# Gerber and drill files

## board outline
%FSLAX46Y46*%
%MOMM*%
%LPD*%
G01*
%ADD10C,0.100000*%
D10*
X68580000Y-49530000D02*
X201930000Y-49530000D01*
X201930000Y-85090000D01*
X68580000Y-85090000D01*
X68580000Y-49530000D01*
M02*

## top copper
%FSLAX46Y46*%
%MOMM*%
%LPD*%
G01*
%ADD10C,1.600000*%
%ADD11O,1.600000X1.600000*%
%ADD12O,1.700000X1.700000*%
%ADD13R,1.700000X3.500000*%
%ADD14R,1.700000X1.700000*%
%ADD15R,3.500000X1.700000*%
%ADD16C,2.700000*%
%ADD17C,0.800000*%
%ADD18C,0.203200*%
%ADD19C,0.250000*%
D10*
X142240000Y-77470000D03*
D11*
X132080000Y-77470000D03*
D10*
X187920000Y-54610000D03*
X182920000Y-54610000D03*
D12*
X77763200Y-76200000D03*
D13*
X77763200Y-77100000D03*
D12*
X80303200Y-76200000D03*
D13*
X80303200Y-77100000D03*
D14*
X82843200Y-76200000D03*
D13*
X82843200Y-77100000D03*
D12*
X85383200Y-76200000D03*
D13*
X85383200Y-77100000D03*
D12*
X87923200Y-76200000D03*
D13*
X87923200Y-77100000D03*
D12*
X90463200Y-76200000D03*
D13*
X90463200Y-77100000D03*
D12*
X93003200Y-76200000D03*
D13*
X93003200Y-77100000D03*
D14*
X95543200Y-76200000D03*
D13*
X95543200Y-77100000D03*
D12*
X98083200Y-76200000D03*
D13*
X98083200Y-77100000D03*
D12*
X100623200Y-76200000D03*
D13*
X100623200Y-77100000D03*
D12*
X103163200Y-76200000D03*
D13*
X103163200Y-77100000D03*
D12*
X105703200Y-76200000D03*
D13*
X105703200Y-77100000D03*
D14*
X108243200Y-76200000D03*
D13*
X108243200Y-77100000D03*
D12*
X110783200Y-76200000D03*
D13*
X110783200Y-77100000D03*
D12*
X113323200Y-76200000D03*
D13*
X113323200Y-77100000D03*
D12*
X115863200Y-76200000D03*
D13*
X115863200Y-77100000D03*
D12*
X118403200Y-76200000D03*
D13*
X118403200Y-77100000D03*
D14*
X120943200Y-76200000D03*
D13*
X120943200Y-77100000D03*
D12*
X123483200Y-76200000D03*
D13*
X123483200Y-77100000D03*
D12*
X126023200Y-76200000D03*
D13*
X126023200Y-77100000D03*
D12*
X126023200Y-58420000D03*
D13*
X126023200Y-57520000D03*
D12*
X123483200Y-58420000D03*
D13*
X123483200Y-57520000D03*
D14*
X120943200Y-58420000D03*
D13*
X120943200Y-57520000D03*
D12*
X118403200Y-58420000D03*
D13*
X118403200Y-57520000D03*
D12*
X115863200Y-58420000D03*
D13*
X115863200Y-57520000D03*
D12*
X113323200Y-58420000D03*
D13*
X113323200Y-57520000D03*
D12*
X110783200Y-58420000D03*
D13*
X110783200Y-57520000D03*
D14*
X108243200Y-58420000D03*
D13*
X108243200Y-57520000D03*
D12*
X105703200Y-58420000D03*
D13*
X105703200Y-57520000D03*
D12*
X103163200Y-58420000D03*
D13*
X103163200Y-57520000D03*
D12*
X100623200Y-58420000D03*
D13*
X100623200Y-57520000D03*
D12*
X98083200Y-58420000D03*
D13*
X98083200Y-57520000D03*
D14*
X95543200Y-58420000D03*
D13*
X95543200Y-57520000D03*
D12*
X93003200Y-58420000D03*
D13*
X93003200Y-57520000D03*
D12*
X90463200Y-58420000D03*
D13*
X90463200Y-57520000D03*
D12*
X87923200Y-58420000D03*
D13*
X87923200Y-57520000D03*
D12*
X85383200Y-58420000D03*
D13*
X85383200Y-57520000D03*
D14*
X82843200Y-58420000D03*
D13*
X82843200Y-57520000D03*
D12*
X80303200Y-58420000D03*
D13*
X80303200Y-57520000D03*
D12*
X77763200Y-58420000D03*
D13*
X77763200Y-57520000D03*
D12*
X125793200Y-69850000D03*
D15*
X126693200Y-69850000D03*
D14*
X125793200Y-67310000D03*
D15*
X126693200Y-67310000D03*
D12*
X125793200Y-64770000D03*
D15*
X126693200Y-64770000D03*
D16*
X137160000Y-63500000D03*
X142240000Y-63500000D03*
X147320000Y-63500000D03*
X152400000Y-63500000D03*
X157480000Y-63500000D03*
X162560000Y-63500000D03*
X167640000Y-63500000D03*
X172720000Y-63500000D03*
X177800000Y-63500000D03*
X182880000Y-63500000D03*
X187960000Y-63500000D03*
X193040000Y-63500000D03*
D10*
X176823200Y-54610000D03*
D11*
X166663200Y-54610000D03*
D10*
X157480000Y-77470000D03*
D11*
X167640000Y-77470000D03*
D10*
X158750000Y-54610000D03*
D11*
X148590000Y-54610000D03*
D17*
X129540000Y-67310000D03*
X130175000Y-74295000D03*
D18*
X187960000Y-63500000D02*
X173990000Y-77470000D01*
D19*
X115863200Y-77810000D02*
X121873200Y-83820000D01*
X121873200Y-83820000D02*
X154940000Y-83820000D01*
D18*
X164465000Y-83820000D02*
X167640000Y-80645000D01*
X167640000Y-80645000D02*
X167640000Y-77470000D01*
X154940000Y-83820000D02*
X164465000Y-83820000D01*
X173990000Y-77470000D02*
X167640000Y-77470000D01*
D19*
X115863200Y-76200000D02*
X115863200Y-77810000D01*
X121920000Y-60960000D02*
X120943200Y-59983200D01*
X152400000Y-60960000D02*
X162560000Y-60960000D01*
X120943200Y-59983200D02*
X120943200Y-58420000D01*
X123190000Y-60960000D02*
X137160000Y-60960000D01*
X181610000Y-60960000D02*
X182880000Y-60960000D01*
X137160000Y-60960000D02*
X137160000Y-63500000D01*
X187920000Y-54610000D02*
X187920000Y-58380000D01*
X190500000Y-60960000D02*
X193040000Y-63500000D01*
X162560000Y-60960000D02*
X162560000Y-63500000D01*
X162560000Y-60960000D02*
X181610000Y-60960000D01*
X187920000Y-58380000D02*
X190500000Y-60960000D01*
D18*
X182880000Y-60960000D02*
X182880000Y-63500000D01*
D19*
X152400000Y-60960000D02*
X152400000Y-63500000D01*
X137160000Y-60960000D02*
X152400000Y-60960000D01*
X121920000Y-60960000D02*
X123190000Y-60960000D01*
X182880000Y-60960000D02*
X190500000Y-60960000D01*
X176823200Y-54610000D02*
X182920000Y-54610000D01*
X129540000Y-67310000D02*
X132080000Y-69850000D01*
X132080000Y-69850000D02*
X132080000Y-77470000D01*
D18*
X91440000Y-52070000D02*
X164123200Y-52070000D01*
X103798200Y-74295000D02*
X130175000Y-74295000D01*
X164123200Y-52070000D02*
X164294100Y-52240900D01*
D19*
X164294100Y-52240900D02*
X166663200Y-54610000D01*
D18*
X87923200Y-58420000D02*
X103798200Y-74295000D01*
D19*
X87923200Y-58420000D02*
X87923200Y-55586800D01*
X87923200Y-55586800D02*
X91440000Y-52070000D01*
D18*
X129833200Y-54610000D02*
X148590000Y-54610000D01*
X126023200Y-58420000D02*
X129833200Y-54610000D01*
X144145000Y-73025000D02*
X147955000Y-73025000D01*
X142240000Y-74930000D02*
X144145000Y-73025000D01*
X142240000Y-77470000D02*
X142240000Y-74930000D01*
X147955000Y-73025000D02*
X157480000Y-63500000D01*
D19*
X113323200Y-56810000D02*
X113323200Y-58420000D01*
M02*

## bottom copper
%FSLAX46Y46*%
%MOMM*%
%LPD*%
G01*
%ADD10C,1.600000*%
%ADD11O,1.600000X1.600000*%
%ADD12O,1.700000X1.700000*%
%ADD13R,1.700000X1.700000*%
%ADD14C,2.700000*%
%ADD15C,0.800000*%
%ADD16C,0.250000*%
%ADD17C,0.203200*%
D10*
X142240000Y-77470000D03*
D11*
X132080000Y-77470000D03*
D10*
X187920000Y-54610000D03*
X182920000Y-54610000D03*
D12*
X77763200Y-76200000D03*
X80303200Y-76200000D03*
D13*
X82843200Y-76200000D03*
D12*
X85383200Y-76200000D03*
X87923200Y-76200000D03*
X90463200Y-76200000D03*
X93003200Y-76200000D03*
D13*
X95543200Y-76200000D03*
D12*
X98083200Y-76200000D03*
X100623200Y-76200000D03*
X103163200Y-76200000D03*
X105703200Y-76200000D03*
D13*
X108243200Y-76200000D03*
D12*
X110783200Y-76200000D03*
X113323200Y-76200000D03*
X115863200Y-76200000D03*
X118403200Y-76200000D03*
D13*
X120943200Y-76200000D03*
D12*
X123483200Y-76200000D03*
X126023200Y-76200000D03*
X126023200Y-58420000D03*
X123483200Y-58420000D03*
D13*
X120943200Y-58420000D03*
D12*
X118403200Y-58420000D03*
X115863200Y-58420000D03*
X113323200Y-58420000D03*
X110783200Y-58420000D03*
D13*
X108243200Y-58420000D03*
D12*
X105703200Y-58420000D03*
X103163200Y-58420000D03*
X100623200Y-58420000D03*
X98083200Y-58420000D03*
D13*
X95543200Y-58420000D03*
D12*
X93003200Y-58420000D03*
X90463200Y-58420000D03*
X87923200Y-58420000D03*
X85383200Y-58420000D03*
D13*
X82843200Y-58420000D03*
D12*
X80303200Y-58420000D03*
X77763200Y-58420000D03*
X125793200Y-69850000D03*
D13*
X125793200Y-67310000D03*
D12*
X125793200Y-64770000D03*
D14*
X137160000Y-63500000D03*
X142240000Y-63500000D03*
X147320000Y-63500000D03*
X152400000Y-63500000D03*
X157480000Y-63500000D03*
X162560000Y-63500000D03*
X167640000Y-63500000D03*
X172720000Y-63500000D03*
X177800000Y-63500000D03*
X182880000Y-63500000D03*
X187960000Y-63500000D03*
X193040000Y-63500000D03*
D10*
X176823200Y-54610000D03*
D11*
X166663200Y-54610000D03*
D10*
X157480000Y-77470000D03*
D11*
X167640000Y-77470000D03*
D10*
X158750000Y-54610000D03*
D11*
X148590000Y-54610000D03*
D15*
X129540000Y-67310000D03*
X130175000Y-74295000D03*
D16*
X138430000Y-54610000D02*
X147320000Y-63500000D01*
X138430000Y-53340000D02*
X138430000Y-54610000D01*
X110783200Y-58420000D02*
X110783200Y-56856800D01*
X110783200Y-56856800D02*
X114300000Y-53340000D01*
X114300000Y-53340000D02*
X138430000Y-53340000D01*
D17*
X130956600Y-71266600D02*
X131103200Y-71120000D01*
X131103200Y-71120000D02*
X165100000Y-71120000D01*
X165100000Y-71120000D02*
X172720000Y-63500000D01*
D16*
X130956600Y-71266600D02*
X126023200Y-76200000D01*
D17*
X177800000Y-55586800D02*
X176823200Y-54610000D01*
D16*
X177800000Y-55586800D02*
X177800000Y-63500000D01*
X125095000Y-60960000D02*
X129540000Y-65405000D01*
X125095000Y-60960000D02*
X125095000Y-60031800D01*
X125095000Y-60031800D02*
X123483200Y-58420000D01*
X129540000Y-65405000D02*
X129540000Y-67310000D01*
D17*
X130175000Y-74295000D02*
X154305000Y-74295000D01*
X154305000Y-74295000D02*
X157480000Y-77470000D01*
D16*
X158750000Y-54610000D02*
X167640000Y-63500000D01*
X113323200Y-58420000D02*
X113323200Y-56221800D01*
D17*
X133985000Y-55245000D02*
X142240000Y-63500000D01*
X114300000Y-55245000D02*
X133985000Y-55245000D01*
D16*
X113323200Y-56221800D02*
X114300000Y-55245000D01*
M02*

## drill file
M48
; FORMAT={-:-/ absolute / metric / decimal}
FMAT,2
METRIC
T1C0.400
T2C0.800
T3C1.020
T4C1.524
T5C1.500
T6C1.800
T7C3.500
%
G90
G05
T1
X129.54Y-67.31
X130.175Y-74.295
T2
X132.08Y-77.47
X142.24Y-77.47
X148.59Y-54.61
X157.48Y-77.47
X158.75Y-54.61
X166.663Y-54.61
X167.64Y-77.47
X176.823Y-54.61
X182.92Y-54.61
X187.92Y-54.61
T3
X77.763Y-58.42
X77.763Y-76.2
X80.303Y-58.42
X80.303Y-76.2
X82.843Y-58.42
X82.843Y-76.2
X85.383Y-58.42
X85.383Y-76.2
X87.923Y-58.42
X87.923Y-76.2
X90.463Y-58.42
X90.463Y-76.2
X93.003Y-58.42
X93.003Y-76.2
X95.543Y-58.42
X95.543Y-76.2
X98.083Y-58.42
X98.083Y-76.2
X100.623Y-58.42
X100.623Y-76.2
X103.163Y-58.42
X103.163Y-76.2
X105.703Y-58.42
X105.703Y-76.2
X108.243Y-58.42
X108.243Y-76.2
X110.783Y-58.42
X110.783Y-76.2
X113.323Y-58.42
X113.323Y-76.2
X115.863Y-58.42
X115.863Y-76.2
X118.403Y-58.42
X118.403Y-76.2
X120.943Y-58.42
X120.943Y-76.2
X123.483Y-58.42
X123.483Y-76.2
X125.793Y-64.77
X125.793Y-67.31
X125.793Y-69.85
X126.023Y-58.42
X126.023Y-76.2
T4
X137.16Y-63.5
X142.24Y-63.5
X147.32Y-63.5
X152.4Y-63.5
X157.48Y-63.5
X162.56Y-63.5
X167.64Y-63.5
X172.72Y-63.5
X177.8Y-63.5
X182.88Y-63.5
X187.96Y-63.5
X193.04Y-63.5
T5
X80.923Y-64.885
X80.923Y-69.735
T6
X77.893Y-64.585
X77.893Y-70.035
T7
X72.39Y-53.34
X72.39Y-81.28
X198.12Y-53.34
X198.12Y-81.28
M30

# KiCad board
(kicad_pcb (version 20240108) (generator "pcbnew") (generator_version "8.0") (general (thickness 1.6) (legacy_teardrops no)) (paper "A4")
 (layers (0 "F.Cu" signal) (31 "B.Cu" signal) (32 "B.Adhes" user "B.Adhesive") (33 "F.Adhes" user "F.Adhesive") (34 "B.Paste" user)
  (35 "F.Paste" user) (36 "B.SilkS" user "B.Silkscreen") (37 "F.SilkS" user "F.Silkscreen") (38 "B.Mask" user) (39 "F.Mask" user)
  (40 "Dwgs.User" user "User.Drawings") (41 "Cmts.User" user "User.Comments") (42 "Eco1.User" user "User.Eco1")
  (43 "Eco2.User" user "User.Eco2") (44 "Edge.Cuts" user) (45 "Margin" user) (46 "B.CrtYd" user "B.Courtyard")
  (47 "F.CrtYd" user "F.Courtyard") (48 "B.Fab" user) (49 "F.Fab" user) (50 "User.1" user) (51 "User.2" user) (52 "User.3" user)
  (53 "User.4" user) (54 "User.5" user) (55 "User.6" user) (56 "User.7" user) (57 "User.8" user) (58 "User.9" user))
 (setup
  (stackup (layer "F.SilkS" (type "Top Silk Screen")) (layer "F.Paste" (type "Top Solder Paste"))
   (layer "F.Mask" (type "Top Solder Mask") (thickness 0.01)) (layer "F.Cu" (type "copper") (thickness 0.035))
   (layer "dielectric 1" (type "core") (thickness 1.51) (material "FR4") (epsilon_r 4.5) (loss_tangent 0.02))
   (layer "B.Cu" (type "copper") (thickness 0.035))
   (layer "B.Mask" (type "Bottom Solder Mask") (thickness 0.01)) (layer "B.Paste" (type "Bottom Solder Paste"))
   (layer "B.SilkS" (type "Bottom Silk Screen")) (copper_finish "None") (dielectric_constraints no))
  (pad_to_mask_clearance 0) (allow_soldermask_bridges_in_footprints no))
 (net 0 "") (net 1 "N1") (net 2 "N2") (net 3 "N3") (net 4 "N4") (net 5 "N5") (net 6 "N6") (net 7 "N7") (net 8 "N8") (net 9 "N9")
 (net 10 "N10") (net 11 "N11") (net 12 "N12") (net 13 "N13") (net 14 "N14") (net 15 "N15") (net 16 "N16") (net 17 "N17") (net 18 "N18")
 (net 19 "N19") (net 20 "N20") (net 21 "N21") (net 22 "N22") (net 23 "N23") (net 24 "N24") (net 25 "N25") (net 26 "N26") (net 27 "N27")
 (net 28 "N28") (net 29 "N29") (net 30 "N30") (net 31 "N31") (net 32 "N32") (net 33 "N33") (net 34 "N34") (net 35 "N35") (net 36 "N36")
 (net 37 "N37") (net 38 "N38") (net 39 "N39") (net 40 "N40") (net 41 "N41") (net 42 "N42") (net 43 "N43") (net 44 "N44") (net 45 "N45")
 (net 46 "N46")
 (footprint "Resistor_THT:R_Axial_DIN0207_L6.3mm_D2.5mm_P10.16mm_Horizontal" (layer "F.Cu") (at 142.24 77.47 180)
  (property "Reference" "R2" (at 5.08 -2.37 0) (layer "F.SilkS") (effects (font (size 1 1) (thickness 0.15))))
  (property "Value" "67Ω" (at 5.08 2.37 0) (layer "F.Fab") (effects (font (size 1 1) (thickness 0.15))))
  (pad "1" thru_hole circle (at 0 0 180) (size 1.6 1.6) (drill 0.8) (layers "*.Cu" "*.Mask") (remove_unused_layers no) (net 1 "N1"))
  (pad "2" thru_hole oval (at 10.16 0 180) (size 1.6 1.6) (drill 0.8) (layers "*.Cu" "*.Mask") (remove_unused_layers no) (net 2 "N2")))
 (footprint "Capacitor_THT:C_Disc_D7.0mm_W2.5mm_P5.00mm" (layer "F.Cu") (at 187.92 54.61 180)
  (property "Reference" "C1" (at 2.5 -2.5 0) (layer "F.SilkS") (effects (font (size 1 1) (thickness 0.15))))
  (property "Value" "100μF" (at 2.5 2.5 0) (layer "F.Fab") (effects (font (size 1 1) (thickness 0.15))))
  (pad "1" thru_hole circle (at 0 0 180) (size 1.6 1.6) (drill 0.8) (layers "*.Cu" "*.Mask") (remove_unused_layers no) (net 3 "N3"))
  (pad "2" thru_hole circle (at 5 0 180) (size 1.6 1.6) (drill 0.8) (layers "*.Cu" "*.Mask") (remove_unused_layers no) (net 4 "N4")))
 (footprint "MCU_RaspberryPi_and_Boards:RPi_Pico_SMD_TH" (layer "F.Cu") (at 101.8932 67.31 90)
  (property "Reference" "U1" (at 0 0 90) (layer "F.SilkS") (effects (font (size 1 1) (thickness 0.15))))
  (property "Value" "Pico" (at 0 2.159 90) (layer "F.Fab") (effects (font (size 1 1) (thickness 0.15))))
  (pad "" np_thru_hole oval (at -2.725 -24 90) (size 1.8 1.8) (drill 1.8) (layers "*.Cu" "*.Mask"))
  (pad "" np_thru_hole oval (at -2.425 -20.97 90) (size 1.5 1.5) (drill 1.5) (layers "*.Cu" "*.Mask"))
  (pad "" np_thru_hole oval (at 2.425 -20.97 90) (size 1.5 1.5) (drill 1.5) (layers "*.Cu" "*.Mask"))
  (pad "" np_thru_hole oval (at 2.725 -24 90) (size 1.8 1.8) (drill 1.8) (layers "*.Cu" "*.Mask"))
  (pad "1" thru_hole oval (at -8.89 -24.13 90) (size 1.7 1.7) (drill 1.02) (layers "*.Cu" "*.Mask") (remove_unused_layers no) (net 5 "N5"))
  (pad "1" smd rect (at -8.89 -24.13 90) (size 3.5 1.7) (drill (offset -0.9 0)) (layers "F.Cu" "F.Mask") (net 5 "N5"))
  (pad "2" thru_hole oval (at -8.89 -21.59 90) (size 1.7 1.7) (drill 1.02) (layers "*.Cu" "*.Mask") (remove_unused_layers no) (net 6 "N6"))
  (pad "2" smd rect (at -8.89 -21.59 90) (size 3.5 1.7) (drill (offset -0.9 0)) (layers "F.Cu" "F.Mask") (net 6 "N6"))
  (pad "3" thru_hole rect (at -8.89 -19.05 90) (size 1.7 1.7) (drill 1.02) (layers "*.Cu" "*.Mask") (remove_unused_layers no) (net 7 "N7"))
  (pad "3" smd rect (at -8.89 -19.05 90) (size 3.5 1.7) (drill (offset -0.9 0)) (layers "F.Cu" "F.Mask") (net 7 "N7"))
  (pad "4" thru_hole oval (at -8.89 -16.51 90) (size 1.7 1.7) (drill 1.02) (layers "*.Cu" "*.Mask") (remove_unused_layers no) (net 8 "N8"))
  (pad "4" smd rect (at -8.89 -16.51 90) (size 3.5 1.7) (drill (offset -0.9 0)) (layers "F.Cu" "F.Mask") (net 8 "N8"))
  (pad "5" thru_hole oval (at -8.89 -13.97 90) (size 1.7 1.7) (drill 1.02) (layers "*.Cu" "*.Mask") (remove_unused_layers no) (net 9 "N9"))
  (pad "5" smd rect (at -8.89 -13.97 90) (size 3.5 1.7) (drill (offset -0.9 0)) (layers "F.Cu" "F.Mask") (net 9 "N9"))
  (pad "6" thru_hole oval (at -8.89 -11.43 90) (size 1.7 1.7) (drill 1.02) (layers "*.Cu" "*.Mask") (remove_unused_layers no) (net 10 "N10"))
  (pad "6" smd rect (at -8.89 -11.43 90) (size 3.5 1.7) (drill (offset -0.9 0)) (layers "F.Cu" "F.Mask") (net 10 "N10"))
  (pad "7" thru_hole oval (at -8.89 -8.89 90) (size 1.7 1.7) (drill 1.02) (layers "*.Cu" "*.Mask") (remove_unused_layers no) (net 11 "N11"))
  (pad "7" smd rect (at -8.89 -8.89 90) (size 3.5 1.7) (drill (offset -0.9 0)) (layers "F.Cu" "F.Mask") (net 11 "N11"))
  (pad "8" thru_hole rect (at -8.89 -6.35 90) (size 1.7 1.7) (drill 1.02) (layers "*.Cu" "*.Mask") (remove_unused_layers no) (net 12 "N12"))
  (pad "8" smd rect (at -8.89 -6.35 90) (size 3.5 1.7) (drill (offset -0.9 0)) (layers "F.Cu" "F.Mask") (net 12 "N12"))
  (pad "9" thru_hole oval (at -8.89 -3.81 90) (size 1.7 1.7) (drill 1.02) (layers "*.Cu" "*.Mask") (remove_unused_layers no) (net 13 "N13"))
  (pad "9" smd rect (at -8.89 -3.81 90) (size 3.5 1.7) (drill (offset -0.9 0)) (layers "F.Cu" "F.Mask") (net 13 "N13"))
  (pad "10" thru_hole oval (at -8.89 -1.27 90) (size 1.7 1.7) (drill 1.02) (layers "*.Cu" "*.Mask") (remove_unused_layers no) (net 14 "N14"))
  (pad "10" smd rect (at -8.89 -1.27 90) (size 3.5 1.7) (drill (offset -0.9 0)) (layers "F.Cu" "F.Mask") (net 14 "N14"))
  (pad "11" thru_hole oval (at -8.89 1.27 90) (size 1.7 1.7) (drill 1.02) (layers "*.Cu" "*.Mask") (remove_unused_layers no) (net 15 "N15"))
  (pad "11" smd rect (at -8.89 1.27 90) (size 3.5 1.7) (drill (offset -0.9 0)) (layers "F.Cu" "F.Mask") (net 15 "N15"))
  (pad "12" thru_hole oval (at -8.89 3.81 90) (size 1.7 1.7) (drill 1.02) (layers "*.Cu" "*.Mask") (remove_unused_layers no) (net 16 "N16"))
  (pad "12" smd rect (at -8.89 3.81 90) (size 3.5 1.7) (drill (offset -0.9 0)) (layers "F.Cu" "F.Mask") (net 16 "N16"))
  (pad "13" thru_hole rect (at -8.89 6.35 90) (size 1.7 1.7) (drill 1.02) (layers "*.Cu" "*.Mask") (remove_unused_layers no) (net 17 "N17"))
  (pad "13" smd rect (at -8.89 6.35 90) (size 3.5 1.7) (drill (offset -0.9 0)) (layers "F.Cu" "F.Mask") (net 17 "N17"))
  (pad "14" thru_hole oval (at -8.89 8.89 90) (size 1.7 1.7) (drill 1.02) (layers "*.Cu" "*.Mask") (remove_unused_layers no) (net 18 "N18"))
  (pad "14" smd rect (at -8.89 8.89 90) (size 3.5 1.7) (drill (offset -0.9 0)) (layers "F.Cu" "F.Mask") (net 18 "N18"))
  (pad "15" thru_hole oval (at -8.89 11.43 90) (size 1.7 1.7) (drill 1.02) (layers "*.Cu" "*.Mask") (remove_unused_layers no) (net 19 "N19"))
  (pad "15" smd rect (at -8.89 11.43 90) (size 3.5 1.7) (drill (offset -0.9 0)) (layers "F.Cu" "F.Mask") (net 19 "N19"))
  (pad "16" thru_hole oval (at -8.89 13.97 90) (size 1.7 1.7) (drill 1.02) (layers "*.Cu" "*.Mask") (remove_unused_layers no) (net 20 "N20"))
  (pad "16" smd rect (at -8.89 13.97 90) (size 3.5 1.7) (drill (offset -0.9 0)) (layers "F.Cu" "F.Mask") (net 20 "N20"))
  (pad "17" thru_hole oval (at -8.89 16.51 90) (size 1.7 1.7) (drill 1.02) (layers "*.Cu" "*.Mask") (remove_unused_layers no) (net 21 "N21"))
  (pad "17" smd rect (at -8.89 16.51 90) (size 3.5 1.7) (drill (offset -0.9 0)) (layers "F.Cu" "F.Mask") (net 21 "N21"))
  (pad "18" thru_hole rect (at -8.89 19.05 90) (size 1.7 1.7) (drill 1.02) (layers "*.Cu" "*.Mask") (remove_unused_layers no) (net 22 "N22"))
  (pad "18" smd rect (at -8.89 19.05 90) (size 3.5 1.7) (drill (offset -0.9 0)) (layers "F.Cu" "F.Mask") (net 22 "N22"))
  (pad "19" thru_hole oval (at -8.89 21.59 90) (size 1.7 1.7) (drill 1.02) (layers "*.Cu" "*.Mask") (remove_unused_layers no) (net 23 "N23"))
  (pad "19" smd rect (at -8.89 21.59 90) (size 3.5 1.7) (drill (offset -0.9 0)) (layers "F.Cu" "F.Mask") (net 23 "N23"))
  (pad "20" thru_hole oval (at -8.89 24.13 90) (size 1.7 1.7) (drill 1.02) (layers "*.Cu" "*.Mask") (remove_unused_layers no) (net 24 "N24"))
  (pad "20" smd rect (at -8.89 24.13 90) (size 3.5 1.7) (drill (offset -0.9 0)) (layers "F.Cu" "F.Mask") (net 24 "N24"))
  (pad "21" thru_hole oval (at 8.89 24.13 90) (size 1.7 1.7) (drill 1.02) (layers "*.Cu" "*.Mask") (remove_unused_layers no) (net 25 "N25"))
  (pad "21" smd rect (at 8.89 24.13 90) (size 3.5 1.7) (drill (offset 0.9 0)) (layers "F.Cu" "F.Mask") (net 25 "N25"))
  (pad "22" thru_hole oval (at 8.89 21.59 90) (size 1.7 1.7) (drill 1.02) (layers "*.Cu" "*.Mask") (remove_unused_layers no) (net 2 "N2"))
  (pad "22" smd rect (at 8.89 21.59 90) (size 3.5 1.7) (drill (offset 0.9 0)) (layers "F.Cu" "F.Mask") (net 2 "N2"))
  (pad "23" thru_hole rect (at 8.89 19.05 90) (size 1.7 1.7) (drill 1.02) (layers "*.Cu" "*.Mask") (remove_unused_layers no) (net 3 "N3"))
  (pad "23" smd rect (at 8.89 19.05 90) (size 3.5 1.7) (drill (offset 0.9 0)) (layers "F.Cu" "F.Mask") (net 3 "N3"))
  (pad "24" thru_hole oval (at 8.89 16.51 90) (size 1.7 1.7) (drill 1.02) (layers "*.Cu" "*.Mask") (remove_unused_layers no) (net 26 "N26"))
  (pad "24" smd rect (at 8.89 16.51 90) (size 3.5 1.7) (drill (offset 0.9 0)) (layers "F.Cu" "F.Mask") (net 26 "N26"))
  (pad "25" thru_hole oval (at 8.89 13.97 90) (size 1.7 1.7) (drill 1.02) (layers "*.Cu" "*.Mask") (remove_unused_layers no) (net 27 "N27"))
  (pad "25" smd rect (at 8.89 13.97 90) (size 3.5 1.7) (drill (offset 0.9 0)) (layers "F.Cu" "F.Mask") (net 27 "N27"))
  (pad "26" thru_hole oval (at 8.89 11.43 90) (size 1.7 1.7) (drill 1.02) (layers "*.Cu" "*.Mask") (remove_unused_layers no) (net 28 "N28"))
  (pad "26" smd rect (at 8.89 11.43 90) (size 3.5 1.7) (drill (offset 0.9 0)) (layers "F.Cu" "F.Mask") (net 28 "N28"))
  (pad "27" thru_hole oval (at 8.89 8.89 90) (size 1.7 1.7) (drill 1.02) (layers "*.Cu" "*.Mask") (remove_unused_layers no) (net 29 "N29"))
  (pad "27" smd rect (at 8.89 8.89 90) (size 3.5 1.7) (drill (offset 0.9 0)) (layers "F.Cu" "F.Mask") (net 29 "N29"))
  (pad "28" thru_hole rect (at 8.89 6.35 90) (size 1.7 1.7) (drill 1.02) (layers "*.Cu" "*.Mask") (remove_unused_layers no) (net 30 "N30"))
  (pad "28" smd rect (at 8.89 6.35 90) (size 3.5 1.7) (drill (offset 0.9 0)) (layers "F.Cu" "F.Mask") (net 30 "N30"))
  (pad "29" thru_hole oval (at 8.89 3.81 90) (size 1.7 1.7) (drill 1.02) (layers "*.Cu" "*.Mask") (remove_unused_layers no) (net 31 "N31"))
  (pad "29" smd rect (at 8.89 3.81 90) (size 3.5 1.7) (drill (offset 0.9 0)) (layers "F.Cu" "F.Mask") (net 31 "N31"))
  (pad "30" thru_hole oval (at 8.89 1.27 90) (size 1.7 1.7) (drill 1.02) (layers "*.Cu" "*.Mask") (remove_unused_layers no) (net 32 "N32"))
  (pad "30" smd rect (at 8.89 1.27 90) (size 3.5 1.7) (drill (offset 0.9 0)) (layers "F.Cu" "F.Mask") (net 32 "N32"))
  (pad "31" thru_hole oval (at 8.89 -1.27 90) (size 1.7 1.7) (drill 1.02) (layers "*.Cu" "*.Mask") (remove_unused_layers no) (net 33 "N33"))
  (pad "31" smd rect (at 8.89 -1.27 90) (size 3.5 1.7) (drill (offset 0.9 0)) (layers "F.Cu" "F.Mask") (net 33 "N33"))
  (pad "32" thru_hole oval (at 8.89 -3.81 90) (size 1.7 1.7) (drill 1.02) (layers "*.Cu" "*.Mask") (remove_unused_layers no) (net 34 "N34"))
  (pad "32" smd rect (at 8.89 -3.81 90) (size 3.5 1.7) (drill (offset 0.9 0)) (layers "F.Cu" "F.Mask") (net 34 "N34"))
  (pad "33" thru_hole rect (at 8.89 -6.35 90) (size 1.7 1.7) (drill 1.02) (layers "*.Cu" "*.Mask") (remove_unused_layers no) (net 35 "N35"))
  (pad "33" smd rect (at 8.89 -6.35 90) (size 3.5 1.7) (drill (offset 0.9 0)) (layers "F.Cu" "F.Mask") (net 35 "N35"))
  (pad "34" thru_hole oval (at 8.89 -8.89 90) (size 1.7 1.7) (drill 1.02) (layers "*.Cu" "*.Mask") (remove_unused_layers no) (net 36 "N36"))
  (pad "34" smd rect (at 8.89 -8.89 90) (size 3.5 1.7) (drill (offset 0.9 0)) (layers "F.Cu" "F.Mask") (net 36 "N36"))
  (pad "35" thru_hole oval (at 8.89 -11.43 90) (size 1.7 1.7) (drill 1.02) (layers "*.Cu" "*.Mask") (remove_unused_layers no) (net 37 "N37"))
  (pad "35" smd rect (at 8.89 -11.43 90) (size 3.5 1.7) (drill (offset 0.9 0)) (layers "F.Cu" "F.Mask") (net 37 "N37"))
  (pad "36" thru_hole oval (at 8.89 -13.97 90) (size 1.7 1.7) (drill 1.02) (layers "*.Cu" "*.Mask") (remove_unused_layers no) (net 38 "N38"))
  (pad "36" smd rect (at 8.89 -13.97 90) (size 3.5 1.7) (drill (offset 0.9 0)) (layers "F.Cu" "F.Mask") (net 38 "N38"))
  (pad "37" thru_hole oval (at 8.89 -16.51 90) (size 1.7 1.7) (drill 1.02) (layers "*.Cu" "*.Mask") (remove_unused_layers no) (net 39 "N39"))
  (pad "37" smd rect (at 8.89 -16.51 90) (size 3.5 1.7) (drill (offset 0.9 0)) (layers "F.Cu" "F.Mask") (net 39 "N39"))
  (pad "38" thru_hole rect (at 8.89 -19.05 90) (size 1.7 1.7) (drill 1.02) (layers "*.Cu" "*.Mask") (remove_unused_layers no) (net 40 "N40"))
  (pad "38" smd rect (at 8.89 -19.05 90) (size 3.5 1.7) (drill (offset 0.9 0)) (layers "F.Cu" "F.Mask") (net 40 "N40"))
  (pad "39" thru_hole oval (at 8.89 -21.59 90) (size 1.7 1.7) (drill 1.02) (layers "*.Cu" "*.Mask") (remove_unused_layers no) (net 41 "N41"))
  (pad "39" smd rect (at 8.89 -21.59 90) (size 3.5 1.7) (drill (offset 0.9 0)) (layers "F.Cu" "F.Mask") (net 41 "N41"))
  (pad "40" thru_hole oval (at 8.89 -24.13 90) (size 1.7 1.7) (drill 1.02) (layers "*.Cu" "*.Mask") (remove_unused_layers no) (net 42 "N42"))
  (pad "40" smd rect (at 8.89 -24.13 90) (size 3.5 1.7) (drill (offset 0.9 0)) (layers "F.Cu" "F.Mask") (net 42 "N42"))
  (pad "41" thru_hole oval (at -2.54 23.9 90) (size 1.7 1.7) (drill 1.02) (layers "*.Cu" "*.Mask") (remove_unused_layers no) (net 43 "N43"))
  (pad "41" smd rect (at -2.54 23.9 180) (size 3.5 1.7) (drill (offset -0.9 0)) (layers "F.Cu" "F.Mask") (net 43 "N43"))
  (pad "42" thru_hole rect (at 0 23.9 90) (size 1.7 1.7) (drill 1.02) (layers "*.Cu" "*.Mask") (remove_unused_layers no) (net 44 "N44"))
  (pad "42" smd rect (at 0 23.9 180) (size 3.5 1.7) (drill (offset -0.9 0)) (layers "F.Cu" "F.Mask") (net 44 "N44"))
  (pad "43" thru_hole oval (at 2.54 23.9 90) (size 1.7 1.7) (drill 1.02) (layers "*.Cu" "*.Mask") (remove_unused_layers no) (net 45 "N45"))
  (pad "43" smd rect (at 2.54 23.9 180) (size 3.5 1.7) (drill (offset -0.9 0)) (layers "F.Cu" "F.Mask") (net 45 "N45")))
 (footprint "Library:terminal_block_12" (layer "F.Cu") (at 170.18 66.04)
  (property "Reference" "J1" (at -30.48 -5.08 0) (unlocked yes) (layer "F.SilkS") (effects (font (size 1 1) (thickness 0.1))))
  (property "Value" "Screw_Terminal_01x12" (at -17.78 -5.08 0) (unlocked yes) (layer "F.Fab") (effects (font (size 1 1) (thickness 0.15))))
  (pad "1" thru_hole circle (at -33.02 -2.54) (size 2.7 2.7) (drill 1.524) (layers "*.Cu" "*.Mask") (remove_unused_layers no) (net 3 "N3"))
  (pad "2" thru_hole circle (at -27.94 -2.54) (size 2.7 2.7) (drill 1.524) (layers "*.Cu" "*.Mask") (remove_unused_layers no) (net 28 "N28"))
  (pad "3" thru_hole circle (at -22.86 -2.54) (size 2.7 2.7) (drill 1.524) (layers "*.Cu" "*.Mask") (remove_unused_layers no) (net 29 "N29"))
  (pad "4" thru_hole circle (at -17.78 -2.54) (size 2.7 2.7) (drill 1.524) (layers "*.Cu" "*.Mask") (remove_unused_layers no) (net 3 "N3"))
  (pad "5" thru_hole circle (at -12.7 -2.54) (size 2.7 2.7) (drill 1.524) (layers "*.Cu" "*.Mask") (remove_unused_layers no) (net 1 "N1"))
  (pad "6" thru_hole circle (at -7.62 -2.54) (size 2.7 2.7) (drill 1.524) (layers "*.Cu" "*.Mask") (remove_unused_layers no) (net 3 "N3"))
  (pad "7" thru_hole circle (at -2.54 -2.54) (size 2.7 2.7) (drill 1.524) (layers "*.Cu" "*.Mask") (remove_unused_layers no) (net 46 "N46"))
  (pad "8" thru_hole circle (at 2.54 -2.54) (size 2.7 2.7) (drill 1.524) (layers "*.Cu" "*.Mask") (remove_unused_layers no) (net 24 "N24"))
  (pad "9" thru_hole circle (at 7.62 -2.54) (size 2.7 2.7) (drill 1.524) (layers "*.Cu" "*.Mask") (remove_unused_layers no) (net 4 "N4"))
  (pad "10" thru_hole circle (at 12.7 -2.54) (size 2.7 2.7) (drill 1.524) (layers "*.Cu" "*.Mask") (remove_unused_layers no) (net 3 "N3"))
  (pad "11" thru_hole circle (at 17.78 -2.54) (size 2.7 2.7) (drill 1.524) (layers "*.Cu" "*.Mask") (remove_unused_layers no) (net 20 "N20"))
  (pad "12" thru_hole circle (at 22.86 -2.54) (size 2.7 2.7) (drill 1.524) (layers "*.Cu" "*.Mask") (remove_unused_layers no) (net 3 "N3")))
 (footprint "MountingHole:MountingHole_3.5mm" (layer "F.Cu") (at 198.12 81.28)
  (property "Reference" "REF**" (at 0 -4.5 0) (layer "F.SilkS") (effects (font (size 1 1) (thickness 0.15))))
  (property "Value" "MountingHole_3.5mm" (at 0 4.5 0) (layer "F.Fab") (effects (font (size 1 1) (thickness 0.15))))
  (pad "" np_thru_hole circle (at 0 0) (size 3.5 3.5) (drill 3.5) (layers "*.Cu" "*.Mask")))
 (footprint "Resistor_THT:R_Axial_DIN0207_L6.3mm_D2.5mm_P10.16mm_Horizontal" (layer "F.Cu") (at 176.8232 54.61 180)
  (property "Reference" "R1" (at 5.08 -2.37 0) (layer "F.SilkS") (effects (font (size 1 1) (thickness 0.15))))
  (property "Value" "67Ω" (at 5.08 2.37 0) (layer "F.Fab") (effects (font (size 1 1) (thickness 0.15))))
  (pad "1" thru_hole circle (at 0 0 180) (size 1.6 1.6) (drill 0.8) (layers "*.Cu" "*.Mask") (remove_unused_layers no) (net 4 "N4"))
  (pad "2" thru_hole oval (at 10.16 0 180) (size 1.6 1.6) (drill 0.8) (layers "*.Cu" "*.Mask") (remove_unused_layers no) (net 38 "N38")))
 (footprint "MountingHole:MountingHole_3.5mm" (layer "F.Cu") (at 198.12 53.34)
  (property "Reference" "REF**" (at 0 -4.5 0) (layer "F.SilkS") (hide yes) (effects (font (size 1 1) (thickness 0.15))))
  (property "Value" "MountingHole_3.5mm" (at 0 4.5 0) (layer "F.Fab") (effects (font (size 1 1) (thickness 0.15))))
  (pad "" np_thru_hole circle (at 0 0) (size 3.5 3.5) (drill 3.5) (layers "*.Cu" "*.Mask")))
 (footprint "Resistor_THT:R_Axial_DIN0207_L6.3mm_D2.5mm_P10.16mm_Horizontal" (layer "F.Cu") (at 157.48 77.47)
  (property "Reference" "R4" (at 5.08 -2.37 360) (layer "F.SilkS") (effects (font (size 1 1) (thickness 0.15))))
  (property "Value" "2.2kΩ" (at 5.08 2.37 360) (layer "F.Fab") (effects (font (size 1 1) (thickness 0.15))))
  (pad "1" thru_hole circle (at 0 0) (size 1.6 1.6) (drill 0.8) (layers "*.Cu" "*.Mask") (remove_unused_layers no) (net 38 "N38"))
  (pad "2" thru_hole oval (at 10.16 0) (size 1.6 1.6) (drill 0.8) (layers "*.Cu" "*.Mask") (remove_unused_layers no) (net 20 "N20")))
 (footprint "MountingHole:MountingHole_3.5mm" (layer "F.Cu") (at 72.39 81.28)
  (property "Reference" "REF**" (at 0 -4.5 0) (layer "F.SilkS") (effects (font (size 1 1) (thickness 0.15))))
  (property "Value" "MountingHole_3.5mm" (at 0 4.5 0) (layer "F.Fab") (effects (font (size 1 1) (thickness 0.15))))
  (pad "" np_thru_hole circle (at 0 0) (size 3.5 3.5) (drill 3.5) (layers "*.Cu" "*.Mask")))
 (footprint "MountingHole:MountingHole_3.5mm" (layer "F.Cu") (at 72.39 53.34)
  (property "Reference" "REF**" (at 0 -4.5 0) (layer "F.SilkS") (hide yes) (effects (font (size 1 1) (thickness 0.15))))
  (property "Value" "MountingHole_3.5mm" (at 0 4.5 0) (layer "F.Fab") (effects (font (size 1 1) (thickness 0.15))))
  (pad "" np_thru_hole circle (at 0 0) (size 3.5 3.5) (drill 3.5) (layers "*.Cu" "*.Mask")))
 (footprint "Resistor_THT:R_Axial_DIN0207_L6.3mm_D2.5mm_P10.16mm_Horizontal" (layer "F.Cu") (at 158.75 54.61 180)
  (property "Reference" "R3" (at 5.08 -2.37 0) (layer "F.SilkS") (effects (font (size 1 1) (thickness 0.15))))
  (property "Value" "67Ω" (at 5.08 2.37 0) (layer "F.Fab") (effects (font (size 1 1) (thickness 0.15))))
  (pad "1" thru_hole circle (at 0 0 180) (size 1.6 1.6) (drill 0.8) (layers "*.Cu" "*.Mask") (remove_unused_layers no) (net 46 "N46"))
  (pad "2" thru_hole oval (at 10.16 0 180) (size 1.6 1.6) (drill 0.8) (layers "*.Cu" "*.Mask") (remove_unused_layers no) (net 25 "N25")))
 (gr_rect (start 68.58 49.53) (end 201.93 85.09) (stroke (width 0.1) (type default)) (fill none) (layer "Edge.Cuts"))
 (segment (start 187.96 63.5) (end 173.99 77.47) (width 0.2032) (layer "F.Cu") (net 20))
 (segment (start 115.8632 77.81) (end 121.8732 83.82) (width 0.25) (layer "F.Cu") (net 20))
 (segment (start 121.8732 83.82) (end 154.94 83.82) (width 0.25) (layer "F.Cu") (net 20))
 (segment (start 164.465 83.82) (end 167.64 80.645) (width 0.2032) (layer "F.Cu") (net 20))
 (segment (start 167.64 80.645) (end 167.64 77.47) (width 0.2032) (layer "F.Cu") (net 20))
 (segment (start 154.94 83.82) (end 164.465 83.82) (width 0.2032) (layer "F.Cu") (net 20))
 (segment (start 173.99 77.47) (end 167.64 77.47) (width 0.2032) (layer "F.Cu") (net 20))
 (segment (start 115.8632 76.2) (end 115.8632 77.81) (width 0.25) (layer "F.Cu") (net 20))
 (segment (start 121.92 60.96) (end 120.9432 59.9832) (width 0.25) (layer "F.Cu") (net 3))
 (segment (start 152.4 60.96) (end 162.56 60.96) (width 0.25) (layer "F.Cu") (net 3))
 (segment (start 120.9432 59.9832) (end 120.9432 58.42) (width 0.25) (layer "F.Cu") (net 3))
 (segment (start 123.19 60.96) (end 137.16 60.96) (width 0.25) (layer "F.Cu") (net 3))
 (segment (start 181.61 60.96) (end 182.88 60.96) (width 0.25) (layer "F.Cu") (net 3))
 (segment (start 137.16 60.96) (end 137.16 63.5) (width 0.25) (layer "F.Cu") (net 3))
 (segment (start 187.92 54.61) (end 187.92 58.38) (width 0.25) (layer "F.Cu") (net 3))
 (segment (start 190.5 60.96) (end 193.04 63.5) (width 0.25) (layer "F.Cu") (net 3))
 (segment (start 162.56 60.96) (end 162.56 63.5) (width 0.25) (layer "F.Cu") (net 3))
 (segment (start 162.56 60.96) (end 181.61 60.96) (width 0.25) (layer "F.Cu") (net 3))
 (segment (start 187.92 58.38) (end 190.5 60.96) (width 0.25) (layer "F.Cu") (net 3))
 (segment (start 182.88 60.96) (end 182.88 63.5) (width 0.2032) (layer "F.Cu") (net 3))
 (segment (start 152.4 60.96) (end 152.4 63.5) (width 0.25) (layer "F.Cu") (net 3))
 (segment (start 137.16 60.96) (end 152.4 60.96) (width 0.25) (layer "F.Cu") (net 3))
 (segment (start 121.92 60.96) (end 123.19 60.96) (width 0.25) (layer "F.Cu") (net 3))
 (segment (start 182.88 60.96) (end 190.5 60.96) (width 0.25) (layer "F.Cu") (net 3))
 (segment (start 138.43 54.61) (end 147.32 63.5) (width 0.25) (layer "B.Cu") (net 29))
 (segment (start 138.43 53.34) (end 138.43 54.61) (width 0.25) (layer "B.Cu") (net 29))
 (segment (start 110.7832 58.42) (end 110.7832 56.8568) (width 0.25) (layer "B.Cu") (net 29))
 (segment (start 110.7832 56.8568) (end 114.3 53.34) (width 0.25) (layer "B.Cu") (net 29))
 (segment (start 114.3 53.34) (end 138.43 53.34) (width 0.25) (layer "B.Cu") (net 29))
 (segment (start 130.9566 71.2666) (end 131.1032 71.12) (width 0.2032) (layer "B.Cu") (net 24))
 (segment (start 131.1032 71.12) (end 165.1 71.12) (width 0.2032) (layer "B.Cu") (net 24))
 (segment (start 165.1 71.12) (end 172.72 63.5) (width 0.2032) (layer "B.Cu") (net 24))
 (segment (start 130.9566 71.2666) (end 126.0232 76.2) (width 0.25) (layer "B.Cu") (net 24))
 (segment (start 176.8232 54.61) (end 182.92 54.61) (width 0.25) (layer "F.Cu") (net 4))
 (segment (start 177.8 55.5868) (end 176.8232 54.61) (width 0.2032) (layer "B.Cu") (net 4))
 (segment (start 177.8 55.5868) (end 177.8 63.5) (width 0.25) (layer "B.Cu") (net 4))
 (segment (start 129.54 67.31) (end 132.08 69.85) (width 0.25) (layer "F.Cu") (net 2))
 (segment (start 132.08 69.85) (end 132.08 77.47) (width 0.25) (layer "F.Cu") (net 2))
 (via (at 129.54 67.31) (size 0.8) (drill 0.4) (layers "F.Cu" "B.Cu") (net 2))
 (segment (start 125.095 60.96) (end 129.54 65.405) (width 0.25) (layer "B.Cu") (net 2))
 (segment (start 125.095 60.96) (end 125.095 60.0318) (width 0.25) (layer "B.Cu") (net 2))
 (segment (start 125.095 60.0318) (end 123.4832 58.42) (width 0.25) (layer "B.Cu") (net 2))
 (segment (start 129.54 65.405) (end 129.54 67.31) (width 0.25) (layer "B.Cu") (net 2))
 (segment (start 91.44 52.07) (end 164.1232 52.07) (width 0.2032) (layer "F.Cu") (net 38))
 (segment (start 103.7982 74.295) (end 130.175 74.295) (width 0.2032) (layer "F.Cu") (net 38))
 (segment (start 164.1232 52.07) (end 164.2941 52.2409) (width 0.2032) (layer "F.Cu") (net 38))
 (segment (start 164.2941 52.2409) (end 166.6632 54.61) (width 0.25) (layer "F.Cu") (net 38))
 (segment (start 87.9232 58.42) (end 103.7982 74.295) (width 0.2032) (layer "F.Cu") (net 38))
 (segment (start 87.9232 58.42) (end 87.9232 55.5868) (width 0.25) (layer "F.Cu") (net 38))
 (segment (start 87.9232 55.5868) (end 91.44 52.07) (width 0.25) (layer "F.Cu") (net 38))
 (via (at 130.175 74.295) (size 0.8) (drill 0.4) (layers "F.Cu" "B.Cu") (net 38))
 (segment (start 130.175 74.295) (end 154.305 74.295) (width 0.2032) (layer "B.Cu") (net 38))
 (segment (start 154.305 74.295) (end 157.48 77.47) (width 0.2032) (layer "B.Cu") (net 38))
 (segment (start 129.8332 54.61) (end 148.59 54.61) (width 0.2032) (layer "F.Cu") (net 25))
 (segment (start 126.0232 58.42) (end 129.8332 54.61) (width 0.2032) (layer "F.Cu") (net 25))
 (segment (start 158.75 54.61) (end 167.64 63.5) (width 0.25) (layer "B.Cu") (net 46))
 (segment (start 144.145 73.025) (end 147.955 73.025) (width 0.2032) (layer "F.Cu") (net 1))
 (segment (start 142.24 74.93) (end 144.145 73.025) (width 0.2032) (layer "F.Cu") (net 1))
 (segment (start 142.24 77.47) (end 142.24 74.93) (width 0.2032) (layer "F.Cu") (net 1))
 (segment (start 147.955 73.025) (end 157.48 63.5) (width 0.2032) (layer "F.Cu") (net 1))
 (segment (start 113.3232 56.81) (end 113.3232 58.42) (width 0.25) (layer "F.Cu") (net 28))
 (segment (start 113.3232 58.42) (end 113.3232 56.2218) (width 0.25) (layer "B.Cu") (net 28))
 (segment (start 133.985 55.245) (end 142.24 63.5) (width 0.2032) (layer "B.Cu") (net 28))
 (segment (start 114.3 55.245) (end 133.985 55.245) (width 0.2032) (layer "B.Cu") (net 28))
 (segment (start 113.3232 56.2218) (end 114.3 55.245) (width 0.25) (layer "B.Cu") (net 28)))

